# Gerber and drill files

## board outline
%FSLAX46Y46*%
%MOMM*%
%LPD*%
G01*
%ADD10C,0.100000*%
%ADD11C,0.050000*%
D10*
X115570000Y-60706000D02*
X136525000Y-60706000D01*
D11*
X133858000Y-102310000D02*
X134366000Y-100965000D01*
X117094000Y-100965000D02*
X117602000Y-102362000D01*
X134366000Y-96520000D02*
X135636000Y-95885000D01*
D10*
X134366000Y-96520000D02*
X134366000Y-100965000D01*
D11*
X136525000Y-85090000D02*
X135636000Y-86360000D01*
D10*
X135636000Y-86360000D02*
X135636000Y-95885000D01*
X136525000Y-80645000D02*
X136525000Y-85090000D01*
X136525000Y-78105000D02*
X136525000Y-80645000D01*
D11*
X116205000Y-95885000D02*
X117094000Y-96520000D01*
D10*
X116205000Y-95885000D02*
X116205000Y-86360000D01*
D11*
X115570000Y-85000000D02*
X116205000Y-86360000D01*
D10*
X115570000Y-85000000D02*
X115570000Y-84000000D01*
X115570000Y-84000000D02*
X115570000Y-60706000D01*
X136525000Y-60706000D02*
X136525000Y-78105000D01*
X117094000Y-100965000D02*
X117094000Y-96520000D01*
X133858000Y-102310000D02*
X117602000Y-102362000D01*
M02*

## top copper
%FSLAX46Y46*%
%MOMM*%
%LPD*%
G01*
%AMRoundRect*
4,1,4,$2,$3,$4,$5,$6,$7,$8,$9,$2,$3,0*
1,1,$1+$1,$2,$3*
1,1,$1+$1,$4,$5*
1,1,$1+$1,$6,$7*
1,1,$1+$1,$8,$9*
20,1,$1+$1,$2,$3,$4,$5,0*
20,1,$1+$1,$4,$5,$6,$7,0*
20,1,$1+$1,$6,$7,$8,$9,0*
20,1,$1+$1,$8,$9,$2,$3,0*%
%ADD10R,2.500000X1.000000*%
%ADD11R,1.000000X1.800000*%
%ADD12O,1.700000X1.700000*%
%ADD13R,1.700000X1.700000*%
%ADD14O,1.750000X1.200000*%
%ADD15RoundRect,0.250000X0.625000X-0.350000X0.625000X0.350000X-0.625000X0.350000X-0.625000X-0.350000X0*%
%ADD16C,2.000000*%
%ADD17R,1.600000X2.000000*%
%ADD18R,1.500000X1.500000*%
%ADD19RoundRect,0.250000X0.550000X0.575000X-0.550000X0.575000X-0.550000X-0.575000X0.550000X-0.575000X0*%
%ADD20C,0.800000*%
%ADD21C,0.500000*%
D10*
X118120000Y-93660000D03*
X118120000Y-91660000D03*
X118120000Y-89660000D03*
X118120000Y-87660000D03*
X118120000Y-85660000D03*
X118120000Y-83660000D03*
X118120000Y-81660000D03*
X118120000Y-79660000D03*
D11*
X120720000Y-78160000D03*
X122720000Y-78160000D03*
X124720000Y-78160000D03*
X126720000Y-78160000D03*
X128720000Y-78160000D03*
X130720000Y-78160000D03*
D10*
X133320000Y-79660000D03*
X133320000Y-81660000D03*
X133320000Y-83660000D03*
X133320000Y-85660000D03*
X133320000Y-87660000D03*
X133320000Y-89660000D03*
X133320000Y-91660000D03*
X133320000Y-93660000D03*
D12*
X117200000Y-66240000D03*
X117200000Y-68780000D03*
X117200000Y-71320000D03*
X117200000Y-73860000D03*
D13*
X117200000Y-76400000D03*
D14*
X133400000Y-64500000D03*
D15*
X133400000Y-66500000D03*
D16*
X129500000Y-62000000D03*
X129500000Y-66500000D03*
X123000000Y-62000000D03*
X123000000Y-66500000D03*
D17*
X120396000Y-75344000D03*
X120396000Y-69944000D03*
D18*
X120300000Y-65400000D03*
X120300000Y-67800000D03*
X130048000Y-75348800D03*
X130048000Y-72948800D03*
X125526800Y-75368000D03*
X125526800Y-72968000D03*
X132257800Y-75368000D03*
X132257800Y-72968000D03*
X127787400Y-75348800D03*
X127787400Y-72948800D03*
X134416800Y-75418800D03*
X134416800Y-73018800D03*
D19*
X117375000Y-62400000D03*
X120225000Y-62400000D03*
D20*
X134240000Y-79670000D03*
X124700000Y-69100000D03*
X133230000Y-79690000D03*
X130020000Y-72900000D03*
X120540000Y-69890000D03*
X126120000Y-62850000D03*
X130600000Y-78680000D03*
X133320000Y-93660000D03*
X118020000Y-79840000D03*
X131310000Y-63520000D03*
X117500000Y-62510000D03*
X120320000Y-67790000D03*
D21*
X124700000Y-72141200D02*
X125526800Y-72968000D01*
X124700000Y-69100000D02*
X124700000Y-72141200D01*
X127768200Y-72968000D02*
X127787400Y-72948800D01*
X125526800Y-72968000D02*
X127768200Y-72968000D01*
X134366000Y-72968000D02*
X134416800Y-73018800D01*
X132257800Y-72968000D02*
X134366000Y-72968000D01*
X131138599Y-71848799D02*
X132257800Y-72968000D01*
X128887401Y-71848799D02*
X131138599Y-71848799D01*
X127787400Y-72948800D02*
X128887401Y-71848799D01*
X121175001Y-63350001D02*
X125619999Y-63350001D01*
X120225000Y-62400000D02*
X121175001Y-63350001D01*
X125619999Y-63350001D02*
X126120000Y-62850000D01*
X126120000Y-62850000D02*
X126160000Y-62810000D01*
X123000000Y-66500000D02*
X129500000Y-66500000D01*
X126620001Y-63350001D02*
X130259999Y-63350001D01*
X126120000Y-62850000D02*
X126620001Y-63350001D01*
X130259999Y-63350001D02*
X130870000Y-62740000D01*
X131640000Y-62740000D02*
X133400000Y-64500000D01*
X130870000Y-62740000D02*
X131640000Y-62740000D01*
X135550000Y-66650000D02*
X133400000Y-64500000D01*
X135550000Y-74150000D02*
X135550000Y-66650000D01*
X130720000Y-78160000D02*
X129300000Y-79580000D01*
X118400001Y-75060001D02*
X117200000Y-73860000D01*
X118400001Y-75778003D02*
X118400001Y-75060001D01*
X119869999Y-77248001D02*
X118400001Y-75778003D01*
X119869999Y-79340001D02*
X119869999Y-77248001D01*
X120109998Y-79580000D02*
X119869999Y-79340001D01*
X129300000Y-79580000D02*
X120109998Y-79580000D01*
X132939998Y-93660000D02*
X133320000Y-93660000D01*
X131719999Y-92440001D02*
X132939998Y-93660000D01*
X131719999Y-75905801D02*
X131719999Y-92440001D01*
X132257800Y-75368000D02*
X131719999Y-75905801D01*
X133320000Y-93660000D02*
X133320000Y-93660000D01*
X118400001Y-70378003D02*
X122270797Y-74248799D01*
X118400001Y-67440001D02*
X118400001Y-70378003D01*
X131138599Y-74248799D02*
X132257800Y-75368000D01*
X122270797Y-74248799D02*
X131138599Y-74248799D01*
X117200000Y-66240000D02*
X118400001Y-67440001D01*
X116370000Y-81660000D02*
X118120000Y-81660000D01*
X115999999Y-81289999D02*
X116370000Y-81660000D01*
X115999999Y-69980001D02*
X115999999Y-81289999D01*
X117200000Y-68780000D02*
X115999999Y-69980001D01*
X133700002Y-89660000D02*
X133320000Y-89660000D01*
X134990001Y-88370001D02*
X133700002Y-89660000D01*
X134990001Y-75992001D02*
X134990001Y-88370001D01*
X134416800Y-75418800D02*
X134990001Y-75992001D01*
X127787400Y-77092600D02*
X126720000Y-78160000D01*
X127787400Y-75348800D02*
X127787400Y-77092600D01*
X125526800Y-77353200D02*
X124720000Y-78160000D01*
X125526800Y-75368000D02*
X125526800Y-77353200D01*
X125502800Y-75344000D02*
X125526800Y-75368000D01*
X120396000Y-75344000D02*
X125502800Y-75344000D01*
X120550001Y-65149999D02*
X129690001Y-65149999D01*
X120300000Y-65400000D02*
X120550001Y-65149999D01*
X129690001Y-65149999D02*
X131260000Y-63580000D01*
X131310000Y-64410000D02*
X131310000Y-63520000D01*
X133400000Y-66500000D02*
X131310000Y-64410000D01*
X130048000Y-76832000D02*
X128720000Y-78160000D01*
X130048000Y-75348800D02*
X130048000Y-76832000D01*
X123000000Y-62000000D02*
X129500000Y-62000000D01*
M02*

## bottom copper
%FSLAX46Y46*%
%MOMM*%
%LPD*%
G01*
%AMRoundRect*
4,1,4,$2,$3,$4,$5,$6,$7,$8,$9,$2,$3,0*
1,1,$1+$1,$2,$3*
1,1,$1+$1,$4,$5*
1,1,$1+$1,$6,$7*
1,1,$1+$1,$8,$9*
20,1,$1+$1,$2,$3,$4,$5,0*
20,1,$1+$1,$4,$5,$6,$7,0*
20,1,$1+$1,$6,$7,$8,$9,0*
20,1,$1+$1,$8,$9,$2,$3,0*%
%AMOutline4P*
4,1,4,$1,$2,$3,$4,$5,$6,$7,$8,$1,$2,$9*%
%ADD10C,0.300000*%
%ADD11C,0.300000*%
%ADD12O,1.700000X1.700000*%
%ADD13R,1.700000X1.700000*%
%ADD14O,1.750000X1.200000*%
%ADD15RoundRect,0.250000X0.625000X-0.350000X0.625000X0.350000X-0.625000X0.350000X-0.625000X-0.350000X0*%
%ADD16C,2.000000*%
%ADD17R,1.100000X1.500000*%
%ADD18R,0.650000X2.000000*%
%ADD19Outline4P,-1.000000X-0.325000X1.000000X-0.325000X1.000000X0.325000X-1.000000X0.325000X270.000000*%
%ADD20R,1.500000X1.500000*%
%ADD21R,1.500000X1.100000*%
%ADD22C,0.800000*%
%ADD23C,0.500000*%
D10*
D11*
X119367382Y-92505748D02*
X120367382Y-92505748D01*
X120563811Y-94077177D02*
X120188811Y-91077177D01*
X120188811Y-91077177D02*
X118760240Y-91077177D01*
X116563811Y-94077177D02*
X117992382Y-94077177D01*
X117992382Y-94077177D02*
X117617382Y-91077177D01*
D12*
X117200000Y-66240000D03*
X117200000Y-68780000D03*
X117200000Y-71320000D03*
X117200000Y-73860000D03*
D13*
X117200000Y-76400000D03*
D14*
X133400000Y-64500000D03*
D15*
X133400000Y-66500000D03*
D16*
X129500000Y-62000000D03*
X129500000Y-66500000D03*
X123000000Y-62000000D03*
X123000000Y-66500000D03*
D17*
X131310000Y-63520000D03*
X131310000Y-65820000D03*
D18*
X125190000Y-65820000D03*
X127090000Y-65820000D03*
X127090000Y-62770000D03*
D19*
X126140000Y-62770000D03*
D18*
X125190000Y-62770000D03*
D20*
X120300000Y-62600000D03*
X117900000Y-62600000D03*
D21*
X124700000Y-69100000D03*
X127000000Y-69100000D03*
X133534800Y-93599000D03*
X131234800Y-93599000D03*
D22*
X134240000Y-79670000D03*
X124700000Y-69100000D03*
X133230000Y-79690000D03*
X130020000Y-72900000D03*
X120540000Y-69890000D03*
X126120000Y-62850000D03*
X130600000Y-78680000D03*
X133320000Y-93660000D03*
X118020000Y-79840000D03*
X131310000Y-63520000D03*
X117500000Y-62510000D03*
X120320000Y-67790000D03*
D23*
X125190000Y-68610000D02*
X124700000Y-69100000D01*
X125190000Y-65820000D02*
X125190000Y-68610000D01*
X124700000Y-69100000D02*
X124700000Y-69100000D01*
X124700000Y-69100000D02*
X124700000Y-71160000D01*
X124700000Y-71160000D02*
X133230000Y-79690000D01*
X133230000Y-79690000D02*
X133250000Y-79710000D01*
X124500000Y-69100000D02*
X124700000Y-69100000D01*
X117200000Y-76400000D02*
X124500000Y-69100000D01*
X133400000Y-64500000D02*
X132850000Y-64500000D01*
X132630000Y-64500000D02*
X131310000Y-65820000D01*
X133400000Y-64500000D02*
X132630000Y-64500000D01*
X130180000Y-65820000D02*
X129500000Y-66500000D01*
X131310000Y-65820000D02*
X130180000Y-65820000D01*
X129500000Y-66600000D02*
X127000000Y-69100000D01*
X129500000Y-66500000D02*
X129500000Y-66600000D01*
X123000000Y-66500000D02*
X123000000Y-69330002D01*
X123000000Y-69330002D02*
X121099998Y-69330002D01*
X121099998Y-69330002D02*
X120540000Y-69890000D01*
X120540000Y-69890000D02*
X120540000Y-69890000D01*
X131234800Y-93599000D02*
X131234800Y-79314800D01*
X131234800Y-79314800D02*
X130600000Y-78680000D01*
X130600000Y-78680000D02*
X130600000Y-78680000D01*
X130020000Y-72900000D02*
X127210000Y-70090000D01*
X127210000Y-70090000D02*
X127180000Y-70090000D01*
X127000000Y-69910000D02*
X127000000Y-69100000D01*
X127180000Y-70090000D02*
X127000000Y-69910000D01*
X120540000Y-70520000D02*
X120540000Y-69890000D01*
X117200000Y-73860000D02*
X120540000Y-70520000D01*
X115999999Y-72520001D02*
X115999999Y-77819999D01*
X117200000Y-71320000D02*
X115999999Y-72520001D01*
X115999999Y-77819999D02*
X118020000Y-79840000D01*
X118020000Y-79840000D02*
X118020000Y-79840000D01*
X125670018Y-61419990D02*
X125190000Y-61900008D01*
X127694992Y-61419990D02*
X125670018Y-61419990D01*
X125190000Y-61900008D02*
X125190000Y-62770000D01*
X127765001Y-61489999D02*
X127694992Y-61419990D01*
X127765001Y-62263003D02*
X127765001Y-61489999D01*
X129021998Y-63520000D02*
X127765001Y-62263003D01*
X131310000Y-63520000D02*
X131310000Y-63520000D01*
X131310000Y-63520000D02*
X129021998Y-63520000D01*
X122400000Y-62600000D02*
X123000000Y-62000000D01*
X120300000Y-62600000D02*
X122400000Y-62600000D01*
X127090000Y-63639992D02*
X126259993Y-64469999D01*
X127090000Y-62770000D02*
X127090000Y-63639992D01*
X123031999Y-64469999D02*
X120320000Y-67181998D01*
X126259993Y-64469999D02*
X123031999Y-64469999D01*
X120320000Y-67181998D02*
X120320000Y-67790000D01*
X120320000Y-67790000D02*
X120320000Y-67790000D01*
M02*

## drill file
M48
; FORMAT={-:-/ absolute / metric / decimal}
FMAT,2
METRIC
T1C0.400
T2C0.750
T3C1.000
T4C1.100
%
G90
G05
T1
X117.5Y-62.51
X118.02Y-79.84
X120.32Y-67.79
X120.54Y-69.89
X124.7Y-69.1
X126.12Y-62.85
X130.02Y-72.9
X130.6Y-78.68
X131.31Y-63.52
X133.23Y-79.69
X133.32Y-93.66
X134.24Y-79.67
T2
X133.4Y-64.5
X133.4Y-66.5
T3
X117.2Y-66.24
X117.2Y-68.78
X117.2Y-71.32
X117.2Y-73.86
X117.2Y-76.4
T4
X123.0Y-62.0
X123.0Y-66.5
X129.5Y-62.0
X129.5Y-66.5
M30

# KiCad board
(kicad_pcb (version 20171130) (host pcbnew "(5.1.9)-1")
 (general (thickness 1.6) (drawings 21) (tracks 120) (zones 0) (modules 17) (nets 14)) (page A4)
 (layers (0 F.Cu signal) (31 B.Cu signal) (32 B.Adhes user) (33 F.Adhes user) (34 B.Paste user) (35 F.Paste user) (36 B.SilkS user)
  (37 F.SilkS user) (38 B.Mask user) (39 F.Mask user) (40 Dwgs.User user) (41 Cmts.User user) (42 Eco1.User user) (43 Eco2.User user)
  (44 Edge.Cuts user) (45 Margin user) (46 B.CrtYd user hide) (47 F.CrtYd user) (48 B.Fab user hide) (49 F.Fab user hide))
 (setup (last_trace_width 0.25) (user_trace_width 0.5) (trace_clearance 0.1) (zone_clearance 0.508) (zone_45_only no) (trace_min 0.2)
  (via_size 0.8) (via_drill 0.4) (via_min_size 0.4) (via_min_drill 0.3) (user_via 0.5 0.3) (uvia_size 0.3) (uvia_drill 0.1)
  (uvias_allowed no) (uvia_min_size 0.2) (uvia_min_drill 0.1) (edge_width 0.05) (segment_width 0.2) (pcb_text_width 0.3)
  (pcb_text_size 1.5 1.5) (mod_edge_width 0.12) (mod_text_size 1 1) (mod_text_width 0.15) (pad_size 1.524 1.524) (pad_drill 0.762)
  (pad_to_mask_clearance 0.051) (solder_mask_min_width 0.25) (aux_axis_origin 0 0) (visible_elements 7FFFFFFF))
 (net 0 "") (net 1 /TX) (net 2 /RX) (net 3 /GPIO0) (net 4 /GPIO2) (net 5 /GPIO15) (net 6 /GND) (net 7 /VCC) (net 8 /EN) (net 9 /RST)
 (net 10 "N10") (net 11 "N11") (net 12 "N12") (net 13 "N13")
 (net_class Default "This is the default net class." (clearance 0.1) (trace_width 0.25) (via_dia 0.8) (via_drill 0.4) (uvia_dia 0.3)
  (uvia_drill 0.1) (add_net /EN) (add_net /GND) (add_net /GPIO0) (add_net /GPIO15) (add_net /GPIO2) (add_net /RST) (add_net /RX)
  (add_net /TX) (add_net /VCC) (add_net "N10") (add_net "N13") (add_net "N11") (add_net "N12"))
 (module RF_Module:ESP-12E (layer F.Cu) (at 125.72 90.16 180)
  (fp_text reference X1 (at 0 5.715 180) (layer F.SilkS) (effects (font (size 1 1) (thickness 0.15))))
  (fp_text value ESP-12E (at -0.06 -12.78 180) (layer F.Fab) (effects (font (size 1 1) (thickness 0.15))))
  (pad 22 smd rect (at 7.6 -3.5 180) (size 2.5 1) (layers F.Cu F.Paste F.Mask))
  (pad 21 smd rect (at 7.6 -1.5 180) (size 2.5 1) (layers F.Cu F.Paste F.Mask))
  (pad 20 smd rect (at 7.6 0.5 180) (size 2.5 1) (layers F.Cu F.Paste F.Mask))
  (pad 19 smd rect (at 7.6 2.5 180) (size 2.5 1) (layers F.Cu F.Paste F.Mask))
  (pad 18 smd rect (at 7.6 4.5 180) (size 2.5 1) (layers F.Cu F.Paste F.Mask))
  (pad 17 smd rect (at 7.6 6.5 180) (size 2.5 1) (layers F.Cu F.Paste F.Mask))
  (pad 16 smd rect (at 7.6 8.5 180) (size 2.5 1) (layers F.Cu F.Paste F.Mask) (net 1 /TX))
  (pad 15 smd rect (at 7.6 10.5 180) (size 2.5 1) (layers F.Cu F.Paste F.Mask) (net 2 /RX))
  (pad 14 smd rect (at 5 12 180) (size 1 1.8) (layers F.Cu F.Paste F.Mask))
  (pad 13 smd rect (at 3 12 180) (size 1 1.8) (layers F.Cu F.Paste F.Mask))
  (pad 12 smd rect (at 1 12 180) (size 1 1.8) (layers F.Cu F.Paste F.Mask) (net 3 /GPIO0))
  (pad 11 smd rect (at -1 12 180) (size 1 1.8) (layers F.Cu F.Paste F.Mask) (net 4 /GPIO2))
  (pad 10 smd rect (at -3 12 180) (size 1 1.8) (layers F.Cu F.Paste F.Mask) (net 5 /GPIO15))
  (pad 9 smd rect (at -5 12 180) (size 1 1.8) (layers F.Cu F.Paste F.Mask) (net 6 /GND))
  (pad 8 smd rect (at -7.6 10.5 180) (size 2.5 1) (layers F.Cu F.Paste F.Mask) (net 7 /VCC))
  (pad 7 smd rect (at -7.6 8.5 180) (size 2.5 1) (layers F.Cu F.Paste F.Mask))
  (pad 6 smd rect (at -7.6 6.5 180) (size 2.5 1) (layers F.Cu F.Paste F.Mask))
  (pad 5 smd rect (at -7.6 4.5 180) (size 2.5 1) (layers F.Cu F.Paste F.Mask))
  (pad 4 smd rect (at -7.6 2.5 180) (size 2.5 1) (layers F.Cu F.Paste F.Mask))
  (pad 3 smd rect (at -7.6 0.5 180) (size 2.5 1) (layers F.Cu F.Paste F.Mask) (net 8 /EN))
  (pad 2 smd rect (at -7.6 -1.5 180) (size 2.5 1) (layers F.Cu F.Paste F.Mask))
  (pad 1 smd rect (at -7.6 -3.5 180) (size 2.5 1) (layers F.Cu F.Paste F.Mask) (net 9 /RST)))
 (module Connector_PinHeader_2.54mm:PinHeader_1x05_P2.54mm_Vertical (layer F.Cu) (at 117.2 76.4 180)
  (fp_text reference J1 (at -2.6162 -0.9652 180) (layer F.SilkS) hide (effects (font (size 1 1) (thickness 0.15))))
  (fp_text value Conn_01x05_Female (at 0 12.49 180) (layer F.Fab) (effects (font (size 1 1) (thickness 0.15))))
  (pad 5 thru_hole oval (at 0 10.16 180) (size 1.7 1.7) (drill 1) (layers *.Cu *.Mask) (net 9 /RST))
  (pad 4 thru_hole oval (at 0 7.62 180) (size 1.7 1.7) (drill 1) (layers *.Cu *.Mask) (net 1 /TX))
  (pad 3 thru_hole oval (at 0 5.08 180) (size 1.7 1.7) (drill 1) (layers *.Cu *.Mask) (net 2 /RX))
  (pad 2 thru_hole oval (at 0 2.54 180) (size 1.7 1.7) (drill 1) (layers *.Cu *.Mask) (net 6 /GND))
  (pad 1 thru_hole rect (at 0 0 180) (size 1.7 1.7) (drill 1) (layers *.Cu *.Mask) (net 7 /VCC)))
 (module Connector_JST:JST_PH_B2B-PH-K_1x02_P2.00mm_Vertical (layer F.Cu) (at 133.4 66.5 90)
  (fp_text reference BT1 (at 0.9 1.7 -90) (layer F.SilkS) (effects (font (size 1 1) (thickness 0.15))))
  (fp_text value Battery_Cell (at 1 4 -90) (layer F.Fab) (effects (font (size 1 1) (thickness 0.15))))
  (pad 2 thru_hole oval (at 2 0 90) (size 1.2 1.75) (drill 0.75) (layers *.Cu *.Mask) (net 6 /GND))
  (pad 1 thru_hole roundrect (at 0 0 90) (size 1.2 1.75) (drill 0.75) (layers *.Cu *.Mask) (roundrect_rratio 0.208333) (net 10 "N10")))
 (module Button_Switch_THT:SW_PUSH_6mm (layer F.Cu) (at 123 62)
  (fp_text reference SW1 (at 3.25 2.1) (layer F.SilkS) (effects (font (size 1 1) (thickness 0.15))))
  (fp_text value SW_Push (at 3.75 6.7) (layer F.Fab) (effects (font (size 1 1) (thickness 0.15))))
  (pad 1 thru_hole circle (at 6.5 0 90) (size 2 2) (drill 1.1) (layers *.Cu *.Mask) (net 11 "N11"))
  (pad 2 thru_hole circle (at 6.5 4.5 90) (size 2 2) (drill 1.1) (layers *.Cu *.Mask) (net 6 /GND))
  (pad 1 thru_hole circle (at 0 0 90) (size 2 2) (drill 1.1) (layers *.Cu *.Mask) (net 11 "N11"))
  (pad 2 thru_hole circle (at 0 4.5 90) (size 2 2) (drill 1.1) (layers *.Cu *.Mask) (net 6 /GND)))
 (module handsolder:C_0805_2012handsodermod (layer B.Cu) (at 131.31 64.67 90)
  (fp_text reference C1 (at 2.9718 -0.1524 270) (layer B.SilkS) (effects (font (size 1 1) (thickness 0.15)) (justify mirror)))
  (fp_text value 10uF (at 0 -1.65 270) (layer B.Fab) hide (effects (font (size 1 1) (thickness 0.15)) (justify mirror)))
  (pad 2 smd rect (at 1.15 0 90) (size 1.5 1.1) (layers B.Cu B.Paste B.Mask) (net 10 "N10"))
  (pad 1 smd rect (at -1.15 0 90) (size 1.5 1.1) (layers B.Cu B.Paste B.Mask) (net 6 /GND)))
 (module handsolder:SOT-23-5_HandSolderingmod (layer B.Cu) (at 126.14 64.32 270)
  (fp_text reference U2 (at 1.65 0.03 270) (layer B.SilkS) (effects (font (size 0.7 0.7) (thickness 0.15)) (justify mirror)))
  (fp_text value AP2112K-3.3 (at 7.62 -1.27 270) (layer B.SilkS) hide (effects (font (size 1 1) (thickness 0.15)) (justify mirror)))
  (pad 5 smd rect (at 1.5 0.95 270) (size 2 0.65) (layers B.Cu B.Paste B.Mask) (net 7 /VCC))
  (pad 4 smd rect (at 1.5 -0.95 270) (size 2 0.65) (layers B.Cu B.Paste B.Mask))
  (pad 3 smd rect (at -1.55 -0.95 270) (size 2 0.65) (layers B.Cu B.Paste B.Mask) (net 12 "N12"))
  (pad 2 smd trapezoid (at -1.55 0 270) (size 2 0.65) (layers B.Cu B.Paste B.Mask) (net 6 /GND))
  (pad 1 smd rect (at -1.55 0.95 270) (size 2 0.65) (layers B.Cu B.Paste B.Mask) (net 10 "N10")))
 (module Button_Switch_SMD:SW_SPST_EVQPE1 (layer F.Cu) (at 120.396 72.644 90)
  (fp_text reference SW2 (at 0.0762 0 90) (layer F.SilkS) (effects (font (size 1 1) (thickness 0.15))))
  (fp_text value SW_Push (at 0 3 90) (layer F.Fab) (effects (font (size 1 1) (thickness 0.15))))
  (pad 1 smd rect (at -2.7 0 90) (size 2 1.6) (layers F.Cu F.Paste F.Mask) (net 3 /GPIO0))
  (pad 2 smd rect (at 2.7 0 90) (size 2 1.6) (layers F.Cu F.Paste F.Mask) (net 6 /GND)))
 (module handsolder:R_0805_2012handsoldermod (layer F.Cu) (at 120.3 66.6 90)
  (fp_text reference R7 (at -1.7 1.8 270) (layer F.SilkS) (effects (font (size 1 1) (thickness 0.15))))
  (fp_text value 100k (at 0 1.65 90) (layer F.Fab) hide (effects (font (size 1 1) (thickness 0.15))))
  (pad 2 smd rect (at 1.2 0 90) (size 1.5 1.5) (layers F.Cu F.Paste F.Mask) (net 10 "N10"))
  (pad 1 smd rect (at -1.2 0 90) (size 1.5 1.5) (layers F.Cu F.Paste F.Mask) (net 12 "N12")))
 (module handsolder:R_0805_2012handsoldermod (layer B.Cu) (at 119.1 62.6)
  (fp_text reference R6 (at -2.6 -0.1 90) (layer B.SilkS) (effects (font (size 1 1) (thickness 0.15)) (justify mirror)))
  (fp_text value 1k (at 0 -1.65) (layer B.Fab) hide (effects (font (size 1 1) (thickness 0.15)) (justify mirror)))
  (pad 2 smd rect (at 1.2 0) (size 1.5 1.5) (layers B.Cu B.Paste B.Mask) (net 11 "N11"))
  (pad 1 smd rect (at -1.2 0) (size 1.5 1.5) (layers B.Cu B.Paste B.Mask) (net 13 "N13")))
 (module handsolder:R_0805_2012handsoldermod (layer F.Cu) (at 130.048 74.1488 270)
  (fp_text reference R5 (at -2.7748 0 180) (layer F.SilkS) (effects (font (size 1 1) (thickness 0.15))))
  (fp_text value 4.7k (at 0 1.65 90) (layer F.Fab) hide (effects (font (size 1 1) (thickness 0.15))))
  (pad 2 smd rect (at 1.2 0 270) (size 1.5 1.5) (layers F.Cu F.Paste F.Mask) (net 5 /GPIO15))
  (pad 1 smd rect (at -1.2 0 270) (size 1.5 1.5) (layers F.Cu F.Paste F.Mask) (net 6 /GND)))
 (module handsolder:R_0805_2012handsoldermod (layer F.Cu) (at 125.5268 74.168 270)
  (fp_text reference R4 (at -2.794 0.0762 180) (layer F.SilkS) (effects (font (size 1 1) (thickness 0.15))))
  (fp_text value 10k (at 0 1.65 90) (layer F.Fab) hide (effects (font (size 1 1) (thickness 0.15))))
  (pad 2 smd rect (at 1.2 0 270) (size 1.5 1.5) (layers F.Cu F.Paste F.Mask) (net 3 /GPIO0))
  (pad 1 smd rect (at -1.2 0 270) (size 1.5 1.5) (layers F.Cu F.Paste F.Mask) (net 7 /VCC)))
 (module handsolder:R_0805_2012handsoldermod (layer F.Cu) (at 132.2578 74.168 270)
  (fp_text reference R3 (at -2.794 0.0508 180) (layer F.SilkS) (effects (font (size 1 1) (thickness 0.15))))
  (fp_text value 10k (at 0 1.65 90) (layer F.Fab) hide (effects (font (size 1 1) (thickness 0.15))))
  (pad 2 smd rect (at 1.2 0 270) (size 1.5 1.5) (layers F.Cu F.Paste F.Mask) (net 9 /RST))
  (pad 1 smd rect (at -1.2 0 270) (size 1.5 1.5) (layers F.Cu F.Paste F.Mask) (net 7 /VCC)))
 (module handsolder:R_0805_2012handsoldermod (layer F.Cu) (at 127.7874 74.1488 270)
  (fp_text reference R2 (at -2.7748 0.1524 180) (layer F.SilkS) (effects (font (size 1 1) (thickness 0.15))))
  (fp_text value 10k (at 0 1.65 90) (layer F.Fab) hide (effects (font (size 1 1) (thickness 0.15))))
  (pad 2 smd rect (at 1.2 0 270) (size 1.5 1.5) (layers F.Cu F.Paste F.Mask) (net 4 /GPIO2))
  (pad 1 smd rect (at -1.2 0 270) (size 1.5 1.5) (layers F.Cu F.Paste F.Mask) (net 7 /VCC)))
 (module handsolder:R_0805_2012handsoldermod (layer F.Cu) (at 134.4168 74.2188 270)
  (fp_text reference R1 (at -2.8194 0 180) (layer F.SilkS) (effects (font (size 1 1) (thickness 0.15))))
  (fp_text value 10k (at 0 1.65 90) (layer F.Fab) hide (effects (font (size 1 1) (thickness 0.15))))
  (pad 2 smd rect (at 1.2 0 270) (size 1.5 1.5) (layers F.Cu F.Paste F.Mask) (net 8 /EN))
  (pad 1 smd rect (at -1.2 0 270) (size 1.5 1.5) (layers F.Cu F.Paste F.Mask) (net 7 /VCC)))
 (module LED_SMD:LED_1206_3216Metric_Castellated (layer F.Cu) (at 118.8 62.4 180)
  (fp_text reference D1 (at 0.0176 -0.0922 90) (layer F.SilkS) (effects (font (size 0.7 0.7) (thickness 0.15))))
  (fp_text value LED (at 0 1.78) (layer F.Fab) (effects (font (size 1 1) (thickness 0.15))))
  (pad 2 smd roundrect (at 1.425 0 180) (size 1.6 1.65) (layers F.Cu F.Paste F.Mask) (roundrect_rratio 0.15625) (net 13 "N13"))
  (pad 1 smd roundrect (at -1.425 0 180) (size 1.6 1.65) (layers F.Cu F.Paste F.Mask) (roundrect_rratio 0.15625) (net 6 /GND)))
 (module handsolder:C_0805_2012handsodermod (layer B.Cu) (at 125.85 69.1 180)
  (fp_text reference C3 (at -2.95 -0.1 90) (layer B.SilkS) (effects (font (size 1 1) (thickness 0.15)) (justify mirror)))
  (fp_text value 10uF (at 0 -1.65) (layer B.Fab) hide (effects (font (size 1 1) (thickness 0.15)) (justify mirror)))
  (pad 2 smd rect (at 1.15 0 180) (size 1.5 1.1) (layers B.Cu B.Paste B.Mask) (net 7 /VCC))
  (pad 1 smd rect (at -1.15 0 180) (size 1.5 1.1) (layers B.Cu B.Paste B.Mask) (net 6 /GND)))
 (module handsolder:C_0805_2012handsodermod (layer B.Cu) (at 132.3848 93.599)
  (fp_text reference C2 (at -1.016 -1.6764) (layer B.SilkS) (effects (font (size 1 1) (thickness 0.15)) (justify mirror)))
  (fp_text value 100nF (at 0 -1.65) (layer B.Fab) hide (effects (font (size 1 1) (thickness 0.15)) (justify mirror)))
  (pad 2 smd rect (at 1.15 0) (size 1.5 1.1) (layers B.Cu B.Paste B.Mask) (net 9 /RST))
  (pad 1 smd rect (at -1.15 0) (size 1.5 1.1) (layers B.Cu B.Paste B.Mask) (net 6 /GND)))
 (gr_line (start 115.57 60.706) (end 136.525 60.706) (layer Edge.Cuts) (width 0.1))
 (gr_line (start 133.858 102.31) (end 134.366 100.965) (layer Edge.Cuts) (width 0.05))
 (gr_line (start 117.094 100.965) (end 117.602 102.362) (layer Edge.Cuts) (width 0.05))
 (gr_line (start 134.366 96.52) (end 135.636 95.885) (layer Edge.Cuts) (width 0.05))
 (gr_line (start 134.366 96.52) (end 134.366 100.965) (layer Edge.Cuts) (width 0.1))
 (gr_line (start 136.525 85.09) (end 135.636 86.36) (layer Edge.Cuts) (width 0.05))
 (gr_line (start 135.636 86.36) (end 135.636 95.885) (layer Edge.Cuts) (width 0.1))
 (gr_line (start 136.525 80.645) (end 136.525 85.09) (layer Edge.Cuts) (width 0.1))
 (gr_line (start 136.525 78.105) (end 136.525 80.645) (layer Edge.Cuts) (width 0.1))
 (gr_line (start 116.205 95.885) (end 117.094 96.52) (layer Edge.Cuts) (width 0.05))
 (gr_line (start 116.205 95.885) (end 116.205 86.36) (layer Edge.Cuts) (width 0.1))
 (gr_line (start 115.57 85) (end 116.205 86.36) (layer Edge.Cuts) (width 0.05))
 (gr_line (start 115.57 85) (end 115.57 84) (layer Edge.Cuts) (width 0.1))
 (gr_line (start 115.57 84) (end 115.57 60.706) (layer Edge.Cuts) (width 0.1))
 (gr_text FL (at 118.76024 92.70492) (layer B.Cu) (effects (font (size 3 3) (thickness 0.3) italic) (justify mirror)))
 (gr_line (start 136.525 60.706) (end 136.525 78.105) (layer Edge.Cuts) (width 0.1))
 (gr_line (start 117.094 100.965) (end 117.094 96.52) (layer Edge.Cuts) (width 0.1))
 (gr_line (start 133.858 102.31) (end 117.602 102.362) (layer Edge.Cuts) (width 0.1))
 (via (at 134.24 79.67) (size 0.8) (drill 0.4) (layers F.Cu B.Cu) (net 7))
 (segment (start 125.19 68.61) (end 124.7 69.1) (width 0.5) (layer B.Cu) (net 7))
 (segment (start 125.19 65.82) (end 125.19 68.61) (width 0.5) (layer B.Cu) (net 7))
 (segment (start 124.7 69.1) (end 124.7 69.1) (width 0.5) (layer B.Cu) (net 7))
 (via (at 124.7 69.1) (size 0.8) (drill 0.4) (layers F.Cu B.Cu) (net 7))
 (segment (start 124.7 72.1412) (end 125.5268 72.968) (width 0.5) (layer F.Cu) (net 7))
 (segment (start 124.7 69.1) (end 124.7 72.1412) (width 0.5) (layer F.Cu) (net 7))
 (segment (start 127.7682 72.968) (end 127.7874 72.9488) (width 0.5) (layer F.Cu) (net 7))
 (segment (start 125.5268 72.968) (end 127.7682 72.968) (width 0.5) (layer F.Cu) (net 7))
 (segment (start 134.366 72.968) (end 134.4168 73.0188) (width 0.5) (layer F.Cu) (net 7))
 (segment (start 132.2578 72.968) (end 134.366 72.968) (width 0.5) (layer F.Cu) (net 7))
 (segment (start 131.138599 71.848799) (end 132.2578 72.968) (width 0.5) (layer F.Cu) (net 7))
 (segment (start 128.887401 71.848799) (end 131.138599 71.848799) (width 0.5) (layer F.Cu) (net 7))
 (segment (start 127.7874 72.9488) (end 128.887401 71.848799) (width 0.5) (layer F.Cu) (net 7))
 (segment (start 124.7 69.1) (end 124.7 71.16) (width 0.5) (layer B.Cu) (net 7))
 (segment (start 124.7 71.16) (end 133.23 79.69) (width 0.5) (layer B.Cu) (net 7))
 (segment (start 133.23 79.69) (end 133.25 79.71) (width 0.5) (layer B.Cu) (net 7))
 (via (at 133.23 79.69) (size 0.8) (drill 0.4) (layers F.Cu B.Cu) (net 7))
 (segment (start 124.5 69.1) (end 124.7 69.1) (width 0.5) (layer B.Cu) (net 7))
 (segment (start 117.2 76.4) (end 124.5 69.1) (width 0.5) (layer B.Cu) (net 7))
 (via (at 130.02 72.9) (size 0.8) (drill 0.4) (layers F.Cu B.Cu) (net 6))
 (segment (start 133.4 64.5) (end 132.85 64.5) (width 0.5) (layer B.Cu) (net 6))
 (segment (start 132.63 64.5) (end 131.31 65.82) (width 0.5) (layer B.Cu) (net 6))
 (segment (start 133.4 64.5) (end 132.63 64.5) (width 0.5) (layer B.Cu) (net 6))
 (segment (start 130.18 65.82) (end 129.5 66.5) (width 0.5) (layer B.Cu) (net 6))
 (segment (start 131.31 65.82) (end 130.18 65.82) (width 0.5) (layer B.Cu) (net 6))
 (segment (start 129.5 66.6) (end 127 69.1) (width 0.5) (layer B.Cu) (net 6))
 (segment (start 129.5 66.5) (end 129.5 66.6) (width 0.5) (layer B.Cu) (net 6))
 (segment (start 123 66.5) (end 123 69.330002) (width 0.5) (layer B.Cu) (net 6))
 (segment (start 123 69.330002) (end 121.099998 69.330002) (width 0.5) (layer B.Cu) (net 6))
 (segment (start 121.099998 69.330002) (end 120.54 69.89) (width 0.5) (layer B.Cu) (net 6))
 (segment (start 120.54 69.89) (end 120.54 69.89) (width 0.5) (layer B.Cu) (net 6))
 (via (at 120.54 69.89) (size 0.8) (drill 0.4) (layers F.Cu B.Cu) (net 6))
 (segment (start 121.175001 63.350001) (end 125.619999 63.350001) (width 0.5) (layer F.Cu) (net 6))
 (segment (start 120.225 62.4) (end 121.175001 63.350001) (width 0.5) (layer F.Cu) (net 6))
 (segment (start 125.619999 63.350001) (end 126.12 62.85) (width 0.5) (layer F.Cu) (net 6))
 (segment (start 126.12 62.85) (end 126.16 62.81) (width 0.5) (layer F.Cu) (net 6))
 (via (at 126.12 62.85) (size 0.8) (drill 0.4) (layers F.Cu B.Cu) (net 6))
 (segment (start 123 66.5) (end 129.5 66.5) (width 0.5) (layer F.Cu) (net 6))
 (segment (start 126.620001 63.350001) (end 130.259999 63.350001) (width 0.5) (layer F.Cu) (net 6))
 (segment (start 126.12 62.85) (end 126.620001 63.350001) (width 0.5) (layer F.Cu) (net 6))
 (segment (start 130.259999 63.350001) (end 130.87 62.74) (width 0.5) (layer F.Cu) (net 6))
 (segment (start 131.64 62.74) (end 133.4 64.5) (width 0.5) (layer F.Cu) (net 6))
 (segment (start 130.87 62.74) (end 131.64 62.74) (width 0.5) (layer F.Cu) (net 6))
 (segment (start 135.55 66.65) (end 133.4 64.5) (width 0.5) (layer F.Cu) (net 6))
 (segment (start 135.55 74.15) (end 135.55 66.65) (width 0.5) (layer F.Cu) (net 6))
 (segment (start 131.2348 93.599) (end 131.2348 79.3148) (width 0.5) (layer B.Cu) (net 6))
 (segment (start 131.2348 79.3148) (end 130.6 78.68) (width 0.5) (layer B.Cu) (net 6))
 (segment (start 130.6 78.68) (end 130.6 78.68) (width 0.5) (layer B.Cu) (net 6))
 (via (at 130.6 78.68) (size 0.8) (drill 0.4) (layers F.Cu B.Cu) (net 6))
 (segment (start 130.72 78.16) (end 129.3 79.58) (width 0.5) (layer F.Cu) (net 6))
 (segment (start 118.400001 75.060001) (end 117.2 73.86) (width 0.5) (layer F.Cu) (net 6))
 (segment (start 118.400001 75.778003) (end 118.400001 75.060001) (width 0.5) (layer F.Cu) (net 6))
 (segment (start 119.869999 77.248001) (end 118.400001 75.778003) (width 0.5) (layer F.Cu) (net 6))
 (segment (start 119.869999 79.340001) (end 119.869999 77.248001) (width 0.5) (layer F.Cu) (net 6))
 (segment (start 120.109998 79.58) (end 119.869999 79.340001) (width 0.5) (layer F.Cu) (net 6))
 (segment (start 129.3 79.58) (end 120.109998 79.58) (width 0.5) (layer F.Cu) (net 6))
 (segment (start 130.02 72.9) (end 127.21 70.09) (width 0.5) (layer B.Cu) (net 6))
 (segment (start 127.21 70.09) (end 127.18 70.09) (width 0.5) (layer B.Cu) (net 6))
 (segment (start 127 69.91) (end 127 69.1) (width 0.5) (layer B.Cu) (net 6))
 (segment (start 127.18 70.09) (end 127 69.91) (width 0.5) (layer B.Cu) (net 6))
 (segment (start 120.54 70.52) (end 120.54 69.89) (width 0.5) (layer B.Cu) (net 6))
 (segment (start 117.2 73.86) (end 120.54 70.52) (width 0.5) (layer B.Cu) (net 6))
 (segment (start 132.939998 93.66) (end 133.32 93.66) (width 0.5) (layer F.Cu) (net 9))
 (segment (start 131.719999 92.440001) (end 132.939998 93.66) (width 0.5) (layer F.Cu) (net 9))
 (segment (start 131.719999 75.905801) (end 131.719999 92.440001) (width 0.5) (layer F.Cu) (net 9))
 (segment (start 132.2578 75.368) (end 131.719999 75.905801) (width 0.5) (layer F.Cu) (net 9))
 (segment (start 133.32 93.66) (end 133.32 93.66) (width 0.5) (layer F.Cu) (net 9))
 (via (at 133.32 93.66) (size 0.8) (drill 0.4) (layers F.Cu B.Cu) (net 9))
 (segment (start 118.400001 70.378003) (end 122.270797 74.248799) (width 0.5) (layer F.Cu) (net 9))
 (segment (start 118.400001 67.440001) (end 118.400001 70.378003) (width 0.5) (layer F.Cu) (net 9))
 (segment (start 131.138599 74.248799) (end 132.2578 75.368) (width 0.5) (layer F.Cu) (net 9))
 (segment (start 122.270797 74.248799) (end 131.138599 74.248799) (width 0.5) (layer F.Cu) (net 9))
 (segment (start 117.2 66.24) (end 118.400001 67.440001) (width 0.5) (layer F.Cu) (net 9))
 (segment (start 115.999999 72.520001) (end 115.999999 77.819999) (width 0.5) (layer B.Cu) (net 2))
 (segment (start 117.2 71.32) (end 115.999999 72.520001) (width 0.5) (layer B.Cu) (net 2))
 (segment (start 115.999999 77.819999) (end 118.02 79.84) (width 0.5) (layer B.Cu) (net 2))
 (segment (start 118.02 79.84) (end 118.02 79.84) (width 0.5) (layer B.Cu) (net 2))
 (via (at 118.02 79.84) (size 0.8) (drill 0.4) (layers F.Cu B.Cu) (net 2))
 (segment (start 116.37 81.66) (end 118.12 81.66) (width 0.5) (layer F.Cu) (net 1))
 (segment (start 115.999999 81.289999) (end 116.37 81.66) (width 0.5) (layer F.Cu) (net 1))
 (segment (start 115.999999 69.980001) (end 115.999999 81.289999) (width 0.5) (layer F.Cu) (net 1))
 (segment (start 117.2 68.78) (end 115.999999 69.980001) (width 0.5) (layer F.Cu) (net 1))
 (segment (start 133.700002 89.66) (end 133.32 89.66) (width 0.5) (layer F.Cu) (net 8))
 (segment (start 134.990001 88.370001) (end 133.700002 89.66) (width 0.5) (layer F.Cu) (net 8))
 (segment (start 134.990001 75.992001) (end 134.990001 88.370001) (width 0.5) (layer F.Cu) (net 8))
 (segment (start 134.4168 75.4188) (end 134.990001 75.992001) (width 0.5) (layer F.Cu) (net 8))
 (segment (start 127.7874 77.0926) (end 126.72 78.16) (width 0.5) (layer F.Cu) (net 4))
 (segment (start 127.7874 75.3488) (end 127.7874 77.0926) (width 0.5) (layer F.Cu) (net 4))
 (segment (start 125.5268 77.3532) (end 124.72 78.16) (width 0.5) (layer F.Cu) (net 3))
 (segment (start 125.5268 75.368) (end 125.5268 77.3532) (width 0.5) (layer F.Cu) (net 3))
 (segment (start 125.5028 75.344) (end 125.5268 75.368) (width 0.5) (layer F.Cu) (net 3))
 (segment (start 120.396 75.344) (end 125.5028 75.344) (width 0.5) (layer F.Cu) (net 3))
 (segment (start 125.670018 61.41999) (end 125.19 61.900008) (width 0.5) (layer B.Cu) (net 10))
 (segment (start 127.694992 61.41999) (end 125.670018 61.41999) (width 0.5) (layer B.Cu) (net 10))
 (segment (start 125.19 61.900008) (end 125.19 62.77) (width 0.5) (layer B.Cu) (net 10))
 (segment (start 127.765001 61.489999) (end 127.694992 61.41999) (width 0.5) (layer B.Cu) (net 10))
 (segment (start 127.765001 62.263003) (end 127.765001 61.489999) (width 0.5) (layer B.Cu) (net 10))
 (segment (start 129.021998 63.52) (end 127.765001 62.263003) (width 0.5) (layer B.Cu) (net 10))
 (segment (start 131.31 63.52) (end 131.31 63.52) (width 0.5) (layer B.Cu) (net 10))
 (segment (start 120.550001 65.149999) (end 129.690001 65.149999) (width 0.5) (layer F.Cu) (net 10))
 (segment (start 120.3 65.4) (end 120.550001 65.149999) (width 0.5) (layer F.Cu) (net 10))
 (segment (start 129.690001 65.149999) (end 131.26 63.58) (width 0.5) (layer F.Cu) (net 10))
 (segment (start 131.31 63.52) (end 129.021998 63.52) (width 0.5) (layer B.Cu) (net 10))
 (via (at 131.31 63.52) (size 0.8) (drill 0.4) (layers F.Cu B.Cu) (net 10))
 (segment (start 131.31 64.41) (end 131.31 63.52) (width 0.5) (layer F.Cu) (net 10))
 (segment (start 133.4 66.5) (end 131.31 64.41) (width 0.5) (layer F.Cu) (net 10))
 (segment (start 130.048 76.832) (end 128.72 78.16) (width 0.5) (layer F.Cu) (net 5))
 (segment (start 130.048 75.3488) (end 130.048 76.832) (width 0.5) (layer F.Cu) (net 5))
 (via (at 117.5 62.51) (size 0.8) (drill 0.4) (layers F.Cu B.Cu) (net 13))
 (segment (start 122.4 62.6) (end 123 62) (width 0.5) (layer B.Cu) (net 11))
 (segment (start 120.3 62.6) (end 122.4 62.6) (width 0.5) (layer B.Cu) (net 11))
 (segment (start 123 62) (end 129.5 62) (width 0.5) (layer F.Cu) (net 11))
 (segment (start 127.09 63.639992) (end 126.259993 64.469999) (width 0.5) (layer B.Cu) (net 12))
 (segment (start 127.09 62.77) (end 127.09 63.639992) (width 0.5) (layer B.Cu) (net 12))
 (segment (start 123.031999 64.469999) (end 120.32 67.181998) (width 0.5) (layer B.Cu) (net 12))
 (segment (start 126.259993 64.469999) (end 123.031999 64.469999) (width 0.5) (layer B.Cu) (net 12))
 (segment (start 120.32 67.181998) (end 120.32 67.79) (width 0.5) (layer B.Cu) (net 12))
 (segment (start 120.32 67.79) (end 120.32 67.79) (width 0.5) (layer B.Cu) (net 12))
 (via (at 120.32 67.79) (size 0.8) (drill 0.4) (layers F.Cu B.Cu) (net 12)))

